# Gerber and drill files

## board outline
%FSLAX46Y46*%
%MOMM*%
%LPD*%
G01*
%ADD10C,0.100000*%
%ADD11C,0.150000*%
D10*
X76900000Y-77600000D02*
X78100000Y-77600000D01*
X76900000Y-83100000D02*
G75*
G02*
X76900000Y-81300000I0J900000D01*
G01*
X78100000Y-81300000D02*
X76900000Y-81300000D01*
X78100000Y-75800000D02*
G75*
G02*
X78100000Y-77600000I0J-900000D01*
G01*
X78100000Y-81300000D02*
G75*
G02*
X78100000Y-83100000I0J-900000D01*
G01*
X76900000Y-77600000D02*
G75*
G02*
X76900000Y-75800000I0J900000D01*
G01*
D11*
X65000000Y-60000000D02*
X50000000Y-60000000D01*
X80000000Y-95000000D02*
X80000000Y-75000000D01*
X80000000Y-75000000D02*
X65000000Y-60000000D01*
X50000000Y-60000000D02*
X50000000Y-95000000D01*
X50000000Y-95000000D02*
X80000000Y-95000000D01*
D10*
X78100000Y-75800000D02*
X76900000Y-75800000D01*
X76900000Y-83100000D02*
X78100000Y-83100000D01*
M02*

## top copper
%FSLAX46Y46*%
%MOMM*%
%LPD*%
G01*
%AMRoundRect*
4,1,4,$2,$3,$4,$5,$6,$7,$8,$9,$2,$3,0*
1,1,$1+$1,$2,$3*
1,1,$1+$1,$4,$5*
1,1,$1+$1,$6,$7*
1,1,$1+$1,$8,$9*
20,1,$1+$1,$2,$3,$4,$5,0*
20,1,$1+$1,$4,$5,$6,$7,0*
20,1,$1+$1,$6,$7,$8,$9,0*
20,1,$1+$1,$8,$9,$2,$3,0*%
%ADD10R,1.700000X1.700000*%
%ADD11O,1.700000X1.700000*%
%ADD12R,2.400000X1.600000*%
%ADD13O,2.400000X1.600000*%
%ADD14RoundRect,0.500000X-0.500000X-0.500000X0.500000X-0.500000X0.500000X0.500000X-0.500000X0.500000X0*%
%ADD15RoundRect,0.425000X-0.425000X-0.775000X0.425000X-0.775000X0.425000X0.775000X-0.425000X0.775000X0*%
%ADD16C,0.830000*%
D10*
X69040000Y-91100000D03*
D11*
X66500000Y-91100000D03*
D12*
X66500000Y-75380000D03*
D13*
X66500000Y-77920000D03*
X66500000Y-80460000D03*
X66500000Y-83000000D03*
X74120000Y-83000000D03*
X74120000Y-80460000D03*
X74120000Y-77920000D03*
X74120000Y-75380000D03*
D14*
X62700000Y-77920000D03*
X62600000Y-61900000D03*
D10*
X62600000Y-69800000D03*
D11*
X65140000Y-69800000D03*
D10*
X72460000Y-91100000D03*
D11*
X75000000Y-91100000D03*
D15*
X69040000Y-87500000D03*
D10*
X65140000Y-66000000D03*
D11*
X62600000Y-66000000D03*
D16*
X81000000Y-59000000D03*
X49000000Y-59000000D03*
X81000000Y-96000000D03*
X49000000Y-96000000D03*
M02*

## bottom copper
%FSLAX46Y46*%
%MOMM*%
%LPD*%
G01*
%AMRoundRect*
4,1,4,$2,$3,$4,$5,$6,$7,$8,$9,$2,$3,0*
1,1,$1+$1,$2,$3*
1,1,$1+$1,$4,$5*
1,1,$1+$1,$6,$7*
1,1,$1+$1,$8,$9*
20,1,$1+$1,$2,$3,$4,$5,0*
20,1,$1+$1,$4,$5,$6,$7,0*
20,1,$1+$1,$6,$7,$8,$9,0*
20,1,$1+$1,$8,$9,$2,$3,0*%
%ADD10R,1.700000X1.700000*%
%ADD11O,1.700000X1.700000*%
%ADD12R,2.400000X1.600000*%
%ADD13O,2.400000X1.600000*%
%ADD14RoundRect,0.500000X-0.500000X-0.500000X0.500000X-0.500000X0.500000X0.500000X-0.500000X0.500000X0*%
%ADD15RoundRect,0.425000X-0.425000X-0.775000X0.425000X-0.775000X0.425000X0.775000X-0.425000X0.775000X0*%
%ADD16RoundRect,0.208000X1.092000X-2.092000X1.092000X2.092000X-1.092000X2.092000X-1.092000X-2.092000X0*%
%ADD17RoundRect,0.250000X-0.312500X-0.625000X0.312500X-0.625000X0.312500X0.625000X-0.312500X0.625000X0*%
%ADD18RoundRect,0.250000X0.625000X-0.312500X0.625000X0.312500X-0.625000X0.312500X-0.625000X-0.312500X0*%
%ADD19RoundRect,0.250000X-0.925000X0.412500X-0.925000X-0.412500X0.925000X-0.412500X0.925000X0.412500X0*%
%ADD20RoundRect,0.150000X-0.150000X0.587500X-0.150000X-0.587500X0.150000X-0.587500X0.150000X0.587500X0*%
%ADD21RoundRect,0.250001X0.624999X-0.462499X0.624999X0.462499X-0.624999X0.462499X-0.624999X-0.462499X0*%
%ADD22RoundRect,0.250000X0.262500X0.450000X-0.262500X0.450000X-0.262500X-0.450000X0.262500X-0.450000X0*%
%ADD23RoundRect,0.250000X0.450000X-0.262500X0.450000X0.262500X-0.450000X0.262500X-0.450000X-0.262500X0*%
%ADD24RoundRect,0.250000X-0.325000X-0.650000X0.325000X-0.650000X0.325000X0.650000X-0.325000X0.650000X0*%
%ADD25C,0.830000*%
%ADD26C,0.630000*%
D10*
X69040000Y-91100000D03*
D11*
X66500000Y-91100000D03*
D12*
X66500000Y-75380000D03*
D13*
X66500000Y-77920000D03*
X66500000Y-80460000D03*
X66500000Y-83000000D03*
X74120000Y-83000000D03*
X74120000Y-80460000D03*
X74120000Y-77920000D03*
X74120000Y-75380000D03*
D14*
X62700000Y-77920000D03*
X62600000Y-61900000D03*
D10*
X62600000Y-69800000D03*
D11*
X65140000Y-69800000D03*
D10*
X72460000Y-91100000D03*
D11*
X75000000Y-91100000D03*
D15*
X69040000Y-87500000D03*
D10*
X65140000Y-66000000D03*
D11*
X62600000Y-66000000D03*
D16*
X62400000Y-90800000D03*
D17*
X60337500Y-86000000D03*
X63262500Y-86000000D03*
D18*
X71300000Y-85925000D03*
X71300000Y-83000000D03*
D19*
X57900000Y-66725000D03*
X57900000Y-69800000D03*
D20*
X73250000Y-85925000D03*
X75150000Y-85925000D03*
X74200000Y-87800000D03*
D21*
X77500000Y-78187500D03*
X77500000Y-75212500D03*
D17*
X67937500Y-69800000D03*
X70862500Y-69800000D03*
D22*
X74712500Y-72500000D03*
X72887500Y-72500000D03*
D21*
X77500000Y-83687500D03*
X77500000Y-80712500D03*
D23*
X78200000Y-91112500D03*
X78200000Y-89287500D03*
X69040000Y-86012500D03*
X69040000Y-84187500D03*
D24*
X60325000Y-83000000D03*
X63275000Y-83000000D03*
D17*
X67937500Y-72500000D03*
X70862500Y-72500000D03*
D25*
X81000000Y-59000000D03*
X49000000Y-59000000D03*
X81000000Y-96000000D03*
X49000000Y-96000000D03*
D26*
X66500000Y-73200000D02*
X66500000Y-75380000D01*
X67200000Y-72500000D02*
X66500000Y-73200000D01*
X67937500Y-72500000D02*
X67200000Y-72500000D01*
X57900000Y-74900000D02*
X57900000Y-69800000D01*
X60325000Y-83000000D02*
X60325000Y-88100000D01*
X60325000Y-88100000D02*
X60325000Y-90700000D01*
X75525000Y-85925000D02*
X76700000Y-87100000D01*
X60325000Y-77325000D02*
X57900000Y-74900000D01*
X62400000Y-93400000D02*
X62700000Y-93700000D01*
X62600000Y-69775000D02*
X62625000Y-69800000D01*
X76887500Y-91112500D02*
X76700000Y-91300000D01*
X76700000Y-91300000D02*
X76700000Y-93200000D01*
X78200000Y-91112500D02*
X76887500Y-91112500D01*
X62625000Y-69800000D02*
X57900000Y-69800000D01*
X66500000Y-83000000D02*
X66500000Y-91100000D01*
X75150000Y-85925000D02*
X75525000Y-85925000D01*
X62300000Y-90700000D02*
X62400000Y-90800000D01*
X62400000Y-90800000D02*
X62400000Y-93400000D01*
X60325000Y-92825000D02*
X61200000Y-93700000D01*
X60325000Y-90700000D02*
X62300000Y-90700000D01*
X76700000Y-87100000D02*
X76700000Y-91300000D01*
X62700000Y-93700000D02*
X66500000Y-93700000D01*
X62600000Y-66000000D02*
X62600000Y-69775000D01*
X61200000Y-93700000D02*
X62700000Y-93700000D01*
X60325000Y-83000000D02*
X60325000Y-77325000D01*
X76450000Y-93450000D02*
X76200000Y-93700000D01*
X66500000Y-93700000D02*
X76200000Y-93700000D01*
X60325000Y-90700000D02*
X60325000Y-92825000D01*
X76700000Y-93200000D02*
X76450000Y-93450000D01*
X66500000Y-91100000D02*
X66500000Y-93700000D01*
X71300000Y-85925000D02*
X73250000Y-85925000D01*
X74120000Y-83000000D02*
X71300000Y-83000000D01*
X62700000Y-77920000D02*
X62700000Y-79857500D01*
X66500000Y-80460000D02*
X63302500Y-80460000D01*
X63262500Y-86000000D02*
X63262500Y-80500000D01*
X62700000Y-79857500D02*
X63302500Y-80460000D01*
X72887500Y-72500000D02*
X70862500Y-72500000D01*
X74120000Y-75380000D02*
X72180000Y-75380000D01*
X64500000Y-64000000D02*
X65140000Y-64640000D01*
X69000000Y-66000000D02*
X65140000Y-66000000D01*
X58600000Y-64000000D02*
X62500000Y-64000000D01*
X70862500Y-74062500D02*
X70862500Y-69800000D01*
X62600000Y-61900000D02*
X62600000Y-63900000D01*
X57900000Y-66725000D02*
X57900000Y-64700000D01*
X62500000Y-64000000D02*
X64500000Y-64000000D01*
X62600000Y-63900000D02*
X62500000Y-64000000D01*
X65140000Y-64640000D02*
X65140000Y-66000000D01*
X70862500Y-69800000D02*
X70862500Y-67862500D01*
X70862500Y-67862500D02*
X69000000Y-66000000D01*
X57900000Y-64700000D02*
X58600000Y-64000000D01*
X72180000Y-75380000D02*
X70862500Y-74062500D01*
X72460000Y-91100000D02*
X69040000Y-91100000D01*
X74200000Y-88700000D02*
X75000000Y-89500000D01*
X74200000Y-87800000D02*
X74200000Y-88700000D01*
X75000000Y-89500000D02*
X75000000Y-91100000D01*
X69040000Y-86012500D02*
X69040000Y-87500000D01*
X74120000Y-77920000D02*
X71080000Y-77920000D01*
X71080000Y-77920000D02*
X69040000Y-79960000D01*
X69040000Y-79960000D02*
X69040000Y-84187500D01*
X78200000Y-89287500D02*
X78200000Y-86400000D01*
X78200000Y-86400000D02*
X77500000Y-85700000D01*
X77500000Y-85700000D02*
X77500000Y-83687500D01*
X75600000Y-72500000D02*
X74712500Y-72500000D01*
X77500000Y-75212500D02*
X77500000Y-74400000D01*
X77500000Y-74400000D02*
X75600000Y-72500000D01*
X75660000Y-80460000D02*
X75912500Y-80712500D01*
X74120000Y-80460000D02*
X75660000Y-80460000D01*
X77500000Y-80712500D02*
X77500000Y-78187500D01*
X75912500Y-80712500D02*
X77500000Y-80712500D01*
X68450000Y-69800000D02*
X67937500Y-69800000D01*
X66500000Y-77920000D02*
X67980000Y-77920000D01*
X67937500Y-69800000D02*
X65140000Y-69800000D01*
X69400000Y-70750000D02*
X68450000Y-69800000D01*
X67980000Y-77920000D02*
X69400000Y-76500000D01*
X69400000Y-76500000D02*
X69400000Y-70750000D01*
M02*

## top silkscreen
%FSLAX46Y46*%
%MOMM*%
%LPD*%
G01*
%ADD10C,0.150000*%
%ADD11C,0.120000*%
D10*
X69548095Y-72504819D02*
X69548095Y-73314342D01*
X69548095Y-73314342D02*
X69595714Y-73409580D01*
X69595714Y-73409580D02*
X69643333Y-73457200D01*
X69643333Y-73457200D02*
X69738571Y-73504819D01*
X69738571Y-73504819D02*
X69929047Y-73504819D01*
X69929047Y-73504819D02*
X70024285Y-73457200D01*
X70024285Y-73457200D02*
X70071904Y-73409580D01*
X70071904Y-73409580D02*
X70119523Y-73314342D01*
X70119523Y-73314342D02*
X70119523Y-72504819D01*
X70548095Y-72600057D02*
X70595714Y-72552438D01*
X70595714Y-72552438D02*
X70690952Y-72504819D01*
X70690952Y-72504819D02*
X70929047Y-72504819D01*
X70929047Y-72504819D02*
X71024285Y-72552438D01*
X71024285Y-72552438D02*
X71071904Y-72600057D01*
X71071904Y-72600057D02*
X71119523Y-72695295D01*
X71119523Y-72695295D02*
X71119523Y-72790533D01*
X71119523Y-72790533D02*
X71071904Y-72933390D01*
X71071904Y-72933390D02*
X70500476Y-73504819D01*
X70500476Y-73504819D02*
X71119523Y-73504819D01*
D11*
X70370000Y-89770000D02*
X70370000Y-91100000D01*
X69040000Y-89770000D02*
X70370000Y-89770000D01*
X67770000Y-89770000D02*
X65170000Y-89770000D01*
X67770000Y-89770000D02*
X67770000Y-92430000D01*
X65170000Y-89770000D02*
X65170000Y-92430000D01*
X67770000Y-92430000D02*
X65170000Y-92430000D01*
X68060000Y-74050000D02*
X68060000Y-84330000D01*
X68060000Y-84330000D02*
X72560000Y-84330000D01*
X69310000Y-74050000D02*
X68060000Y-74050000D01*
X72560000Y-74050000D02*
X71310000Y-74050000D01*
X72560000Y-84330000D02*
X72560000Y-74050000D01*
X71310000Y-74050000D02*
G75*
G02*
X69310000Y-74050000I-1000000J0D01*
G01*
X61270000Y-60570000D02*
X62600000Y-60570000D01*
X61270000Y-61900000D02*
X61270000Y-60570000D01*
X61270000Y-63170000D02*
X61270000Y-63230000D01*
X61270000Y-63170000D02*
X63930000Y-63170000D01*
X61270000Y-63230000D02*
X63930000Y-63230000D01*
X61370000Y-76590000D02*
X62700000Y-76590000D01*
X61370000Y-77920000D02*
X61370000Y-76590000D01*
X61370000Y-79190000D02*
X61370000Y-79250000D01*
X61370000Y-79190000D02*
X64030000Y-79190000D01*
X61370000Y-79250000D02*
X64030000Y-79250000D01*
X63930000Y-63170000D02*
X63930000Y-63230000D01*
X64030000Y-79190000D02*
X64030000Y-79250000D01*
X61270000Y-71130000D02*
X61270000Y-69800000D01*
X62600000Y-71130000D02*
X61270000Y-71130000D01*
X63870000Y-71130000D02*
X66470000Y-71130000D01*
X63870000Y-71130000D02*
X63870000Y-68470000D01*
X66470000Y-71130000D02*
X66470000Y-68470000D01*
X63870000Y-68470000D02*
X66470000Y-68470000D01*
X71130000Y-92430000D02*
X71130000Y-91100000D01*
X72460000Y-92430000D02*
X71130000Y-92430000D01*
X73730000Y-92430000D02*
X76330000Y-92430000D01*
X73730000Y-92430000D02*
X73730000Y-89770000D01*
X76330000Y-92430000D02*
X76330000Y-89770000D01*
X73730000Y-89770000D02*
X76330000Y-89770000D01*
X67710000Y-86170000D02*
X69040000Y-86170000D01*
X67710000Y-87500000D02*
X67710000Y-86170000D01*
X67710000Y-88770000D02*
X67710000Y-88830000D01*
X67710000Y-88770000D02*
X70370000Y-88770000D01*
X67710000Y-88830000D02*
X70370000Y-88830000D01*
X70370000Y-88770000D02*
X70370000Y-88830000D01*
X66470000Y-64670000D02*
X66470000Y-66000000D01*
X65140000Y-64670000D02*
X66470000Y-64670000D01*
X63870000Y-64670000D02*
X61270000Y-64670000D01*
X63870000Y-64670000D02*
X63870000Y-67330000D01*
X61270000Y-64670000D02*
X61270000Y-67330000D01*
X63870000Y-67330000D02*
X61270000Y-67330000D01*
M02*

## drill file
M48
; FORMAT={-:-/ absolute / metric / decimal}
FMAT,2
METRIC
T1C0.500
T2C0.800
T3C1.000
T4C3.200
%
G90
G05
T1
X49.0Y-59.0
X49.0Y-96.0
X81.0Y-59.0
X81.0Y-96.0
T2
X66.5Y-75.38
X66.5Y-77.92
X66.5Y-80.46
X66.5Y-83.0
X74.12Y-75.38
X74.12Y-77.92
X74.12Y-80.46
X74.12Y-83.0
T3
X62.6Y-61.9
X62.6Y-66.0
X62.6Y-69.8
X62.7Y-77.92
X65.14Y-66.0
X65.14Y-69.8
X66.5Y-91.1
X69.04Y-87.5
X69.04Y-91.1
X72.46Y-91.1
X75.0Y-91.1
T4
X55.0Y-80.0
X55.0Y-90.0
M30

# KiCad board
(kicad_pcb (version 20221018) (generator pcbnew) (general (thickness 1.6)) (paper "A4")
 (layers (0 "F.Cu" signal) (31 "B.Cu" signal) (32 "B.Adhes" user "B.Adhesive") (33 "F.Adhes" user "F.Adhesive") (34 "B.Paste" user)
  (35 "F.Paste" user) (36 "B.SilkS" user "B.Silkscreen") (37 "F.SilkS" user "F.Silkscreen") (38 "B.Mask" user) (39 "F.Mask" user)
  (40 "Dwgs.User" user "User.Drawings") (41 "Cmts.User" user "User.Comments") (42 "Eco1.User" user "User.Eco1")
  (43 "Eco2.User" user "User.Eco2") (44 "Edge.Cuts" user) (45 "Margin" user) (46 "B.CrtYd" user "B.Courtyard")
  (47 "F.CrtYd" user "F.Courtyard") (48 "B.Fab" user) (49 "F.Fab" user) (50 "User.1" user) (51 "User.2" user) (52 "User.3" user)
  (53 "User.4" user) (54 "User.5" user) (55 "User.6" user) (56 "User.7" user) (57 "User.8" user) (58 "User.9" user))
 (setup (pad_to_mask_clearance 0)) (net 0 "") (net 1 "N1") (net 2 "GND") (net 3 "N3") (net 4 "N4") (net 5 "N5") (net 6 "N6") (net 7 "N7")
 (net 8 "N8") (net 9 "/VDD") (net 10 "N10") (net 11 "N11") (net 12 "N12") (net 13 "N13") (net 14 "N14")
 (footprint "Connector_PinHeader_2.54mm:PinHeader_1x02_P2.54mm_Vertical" (layer "F.Cu") (at 69.04 91.1 -90)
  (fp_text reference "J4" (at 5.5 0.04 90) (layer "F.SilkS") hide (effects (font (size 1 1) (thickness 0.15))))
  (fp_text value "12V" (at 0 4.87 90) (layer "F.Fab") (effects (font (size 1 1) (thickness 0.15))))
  (fp_line (start -1.33 -1.33) (end 0 -1.33) (stroke (width 0.12) (type solid)) (layer "F.SilkS"))
  (fp_line (start -1.33 0) (end -1.33 -1.33) (stroke (width 0.12) (type solid)) (layer "F.SilkS"))
  (fp_line (start -1.33 1.27) (end -1.33 3.87) (stroke (width 0.12) (type solid)) (layer "F.SilkS"))
  (fp_line (start -1.33 1.27) (end 1.33 1.27) (stroke (width 0.12) (type solid)) (layer "F.SilkS"))
  (fp_line (start -1.33 3.87) (end 1.33 3.87) (stroke (width 0.12) (type solid)) (layer "F.SilkS"))
  (fp_line (start 1.33 1.27) (end 1.33 3.87) (stroke (width 0.12) (type solid)) (layer "F.SilkS"))
  (pad "1" thru_hole rect (at 0 0 270) (size 1.7 1.7) (drill 1) (layers "*.Cu" "*.Mask") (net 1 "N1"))
  (pad "2" thru_hole oval (at 0 2.54 270) (size 1.7 1.7) (drill 1) (layers "*.Cu" "*.Mask") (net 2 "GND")))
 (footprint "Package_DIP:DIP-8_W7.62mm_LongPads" (layer "F.Cu") (at 66.5 75.38)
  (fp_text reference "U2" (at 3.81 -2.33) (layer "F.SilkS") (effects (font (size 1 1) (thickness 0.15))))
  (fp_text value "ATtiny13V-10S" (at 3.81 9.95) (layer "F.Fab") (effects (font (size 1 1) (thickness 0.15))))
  (fp_line (start 1.56 -1.33) (end 1.56 8.95) (stroke (width 0.12) (type solid)) (layer "F.SilkS"))
  (fp_line (start 1.56 8.95) (end 6.06 8.95) (stroke (width 0.12) (type solid)) (layer "F.SilkS"))
  (fp_line (start 2.81 -1.33) (end 1.56 -1.33) (stroke (width 0.12) (type solid)) (layer "F.SilkS"))
  (fp_line (start 6.06 -1.33) (end 4.81 -1.33) (stroke (width 0.12) (type solid)) (layer "F.SilkS"))
  (fp_line (start 6.06 8.95) (end 6.06 -1.33) (stroke (width 0.12) (type solid)) (layer "F.SilkS"))
  (fp_arc (start 4.81 -1.33) (mid 3.81 -0.33) (end 2.81 -1.33) (stroke (width 0.12) (type solid)) (layer "F.SilkS"))
  (pad "1" thru_hole rect (at 0 0) (size 2.4 1.6) (drill 0.8) (layers "*.Cu" "*.Mask") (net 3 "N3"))
  (pad "2" thru_hole oval (at 0 2.54) (size 2.4 1.6) (drill 0.8) (layers "*.Cu" "*.Mask") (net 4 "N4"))
  (pad "3" thru_hole oval (at 0 5.08) (size 2.4 1.6) (drill 0.8) (layers "*.Cu" "*.Mask") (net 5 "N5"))
  (pad "4" thru_hole oval (at 0 7.62) (size 2.4 1.6) (drill 0.8) (layers "*.Cu" "*.Mask") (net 2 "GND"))
  (pad "5" thru_hole oval (at 7.62 7.62) (size 2.4 1.6) (drill 0.8) (layers "*.Cu" "*.Mask") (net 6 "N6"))
  (pad "6" thru_hole oval (at 7.62 5.08) (size 2.4 1.6) (drill 0.8) (layers "*.Cu" "*.Mask") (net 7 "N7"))
  (pad "7" thru_hole oval (at 7.62 2.54) (size 2.4 1.6) (drill 0.8) (layers "*.Cu" "*.Mask") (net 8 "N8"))
  (pad "8" thru_hole oval (at 7.62 0) (size 2.4 1.6) (drill 0.8) (layers "*.Cu" "*.Mask") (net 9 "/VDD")))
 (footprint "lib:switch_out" (layer "F.Cu") (at 62.7 68.92)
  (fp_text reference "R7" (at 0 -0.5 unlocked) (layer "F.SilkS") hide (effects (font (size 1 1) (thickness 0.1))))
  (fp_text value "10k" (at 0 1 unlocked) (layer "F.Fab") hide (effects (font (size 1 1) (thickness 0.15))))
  (fp_line (start -1.43 -8.35) (end -0.1 -8.35) (stroke (width 0.12) (type solid)) (layer "F.SilkS"))
  (fp_line (start -1.43 -7.02) (end -1.43 -8.35) (stroke (width 0.12) (type solid)) (layer "F.SilkS"))
  (fp_line (start -1.43 -5.75) (end -1.43 -5.69) (stroke (width 0.12) (type solid)) (layer "F.SilkS"))
  (fp_line (start -1.43 -5.75) (end 1.23 -5.75) (stroke (width 0.12) (type solid)) (layer "F.SilkS"))
  (fp_line (start -1.43 -5.69) (end 1.23 -5.69) (stroke (width 0.12) (type solid)) (layer "F.SilkS"))
  (fp_line (start -1.33 7.67) (end 0 7.67) (stroke (width 0.12) (type solid)) (layer "F.SilkS"))
  (fp_line (start -1.33 9) (end -1.33 7.67) (stroke (width 0.12) (type solid)) (layer "F.SilkS"))
  (fp_line (start -1.33 10.27) (end -1.33 10.33) (stroke (width 0.12) (type solid)) (layer "F.SilkS"))
  (fp_line (start -1.33 10.27) (end 1.33 10.27) (stroke (width 0.12) (type solid)) (layer "F.SilkS"))
  (fp_line (start -1.33 10.33) (end 1.33 10.33) (stroke (width 0.12) (type solid)) (layer "F.SilkS"))
  (fp_line (start 1.23 -5.75) (end 1.23 -5.69) (stroke (width 0.12) (type solid)) (layer "F.SilkS"))
  (fp_line (start 1.33 10.27) (end 1.33 10.33) (stroke (width 0.12) (type solid)) (layer "F.SilkS"))
  (pad "1" thru_hole roundrect (at 0 9) (size 2 2) (drill 1) (layers "*.Cu" "*.Mask") (roundrect_rratio 0.25) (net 5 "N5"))
  (pad "2" thru_hole roundrect (at -0.1 -7.02) (size 2 2) (drill 1) (layers "*.Cu" "*.Mask") (roundrect_rratio 0.25) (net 9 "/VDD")))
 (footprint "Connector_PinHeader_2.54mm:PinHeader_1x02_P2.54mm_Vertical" (layer "F.Cu") (at 62.6 69.8 90)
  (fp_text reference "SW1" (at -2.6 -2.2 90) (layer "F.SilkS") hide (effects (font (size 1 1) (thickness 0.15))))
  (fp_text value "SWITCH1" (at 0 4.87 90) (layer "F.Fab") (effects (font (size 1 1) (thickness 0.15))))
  (fp_line (start -1.33 -1.33) (end 0 -1.33) (stroke (width 0.12) (type solid)) (layer "F.SilkS"))
  (fp_line (start -1.33 0) (end -1.33 -1.33) (stroke (width 0.12) (type solid)) (layer "F.SilkS"))
  (fp_line (start -1.33 1.27) (end -1.33 3.87) (stroke (width 0.12) (type solid)) (layer "F.SilkS"))
  (fp_line (start -1.33 1.27) (end 1.33 1.27) (stroke (width 0.12) (type solid)) (layer "F.SilkS"))
  (fp_line (start -1.33 3.87) (end 1.33 3.87) (stroke (width 0.12) (type solid)) (layer "F.SilkS"))
  (fp_line (start 1.33 1.27) (end 1.33 3.87) (stroke (width 0.12) (type solid)) (layer "F.SilkS"))
  (pad "1" thru_hole rect (at 0 0 90) (size 1.7 1.7) (drill 1) (layers "*.Cu" "*.Mask") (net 2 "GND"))
  (pad "2" thru_hole oval (at 0 2.54 90) (size 1.7 1.7) (drill 1) (layers "*.Cu" "*.Mask") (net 4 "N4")))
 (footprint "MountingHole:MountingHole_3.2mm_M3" (layer "F.Cu") (at 55 90)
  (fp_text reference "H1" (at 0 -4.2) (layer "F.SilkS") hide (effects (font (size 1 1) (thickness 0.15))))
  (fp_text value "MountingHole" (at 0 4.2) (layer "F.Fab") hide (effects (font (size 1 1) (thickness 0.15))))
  (pad "" np_thru_hole circle (at 0 0) (size 3.2 3.2) (drill 3.2) (layers "*.Cu" "*.Mask")))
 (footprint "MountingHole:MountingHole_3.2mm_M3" (layer "F.Cu") (at 55 80)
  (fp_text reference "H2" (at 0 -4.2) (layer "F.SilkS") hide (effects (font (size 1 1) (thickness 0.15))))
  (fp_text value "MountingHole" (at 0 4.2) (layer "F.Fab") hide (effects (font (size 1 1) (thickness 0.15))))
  (pad "" np_thru_hole circle (at 0 0) (size 3.2 3.2) (drill 3.2) (layers "*.Cu" "*.Mask")))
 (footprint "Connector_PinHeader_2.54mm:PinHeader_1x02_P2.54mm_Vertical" (layer "F.Cu") (at 72.46 91.1 90)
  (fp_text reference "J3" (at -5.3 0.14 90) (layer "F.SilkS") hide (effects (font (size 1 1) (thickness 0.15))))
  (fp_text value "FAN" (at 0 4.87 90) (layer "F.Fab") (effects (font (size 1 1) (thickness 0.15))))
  (fp_line (start -1.33 -1.33) (end 0 -1.33) (stroke (width 0.12) (type solid)) (layer "F.SilkS"))
  (fp_line (start -1.33 0) (end -1.33 -1.33) (stroke (width 0.12) (type solid)) (layer "F.SilkS"))
  (fp_line (start -1.33 1.27) (end -1.33 3.87) (stroke (width 0.12) (type solid)) (layer "F.SilkS"))
  (fp_line (start -1.33 1.27) (end 1.33 1.27) (stroke (width 0.12) (type solid)) (layer "F.SilkS"))
  (fp_line (start -1.33 3.87) (end 1.33 3.87) (stroke (width 0.12) (type solid)) (layer "F.SilkS"))
  (fp_line (start 1.33 1.27) (end 1.33 3.87) (stroke (width 0.12) (type solid)) (layer "F.SilkS"))
  (pad "1" thru_hole rect (at 0 0 90) (size 1.7 1.7) (drill 1) (layers "*.Cu" "*.Mask") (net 1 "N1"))
  (pad "2" thru_hole oval (at 0 2.54 90) (size 1.7 1.7) (drill 1) (layers "*.Cu" "*.Mask") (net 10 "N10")))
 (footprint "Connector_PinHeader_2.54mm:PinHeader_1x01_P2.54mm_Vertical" (layer "F.Cu") (at 69.04 87.5)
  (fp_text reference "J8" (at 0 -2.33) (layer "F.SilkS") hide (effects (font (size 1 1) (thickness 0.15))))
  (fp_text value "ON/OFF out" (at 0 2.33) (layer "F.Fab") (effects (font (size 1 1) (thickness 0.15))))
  (fp_line (start -1.33 -1.33) (end 0 -1.33) (stroke (width 0.12) (type solid)) (layer "F.SilkS"))
  (fp_line (start -1.33 0) (end -1.33 -1.33) (stroke (width 0.12) (type solid)) (layer "F.SilkS"))
  (fp_line (start -1.33 1.27) (end -1.33 1.33) (stroke (width 0.12) (type solid)) (layer "F.SilkS"))
  (fp_line (start -1.33 1.27) (end 1.33 1.27) (stroke (width 0.12) (type solid)) (layer "F.SilkS"))
  (fp_line (start -1.33 1.33) (end 1.33 1.33) (stroke (width 0.12) (type solid)) (layer "F.SilkS"))
  (fp_line (start 1.33 1.27) (end 1.33 1.33) (stroke (width 0.12) (type solid)) (layer "F.SilkS"))
  (pad "1" thru_hole roundrect (at 0 0) (size 1.7 2.4) (drill 1) (layers "*.Cu" "*.Mask") (roundrect_rratio 0.25) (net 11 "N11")))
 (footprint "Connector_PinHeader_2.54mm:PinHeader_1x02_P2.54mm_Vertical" (layer "F.Cu") (at 65.14 66 -90)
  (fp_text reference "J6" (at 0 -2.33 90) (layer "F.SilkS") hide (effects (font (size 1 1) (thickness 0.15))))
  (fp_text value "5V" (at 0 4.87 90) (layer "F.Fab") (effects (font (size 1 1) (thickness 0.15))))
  (fp_line (start -1.33 -1.33) (end 0 -1.33) (stroke (width 0.12) (type solid)) (layer "F.SilkS"))
  (fp_line (start -1.33 0) (end -1.33 -1.33) (stroke (width 0.12) (type solid)) (layer "F.SilkS"))
  (fp_line (start -1.33 1.27) (end -1.33 3.87) (stroke (width 0.12) (type solid)) (layer "F.SilkS"))
  (fp_line (start -1.33 1.27) (end 1.33 1.27) (stroke (width 0.12) (type solid)) (layer "F.SilkS"))
  (fp_line (start -1.33 3.87) (end 1.33 3.87) (stroke (width 0.12) (type solid)) (layer "F.SilkS"))
  (fp_line (start 1.33 1.27) (end 1.33 3.87) (stroke (width 0.12) (type solid)) (layer "F.SilkS"))
  (pad "1" thru_hole rect (at 0 0 270) (size 1.7 1.7) (drill 1) (layers "*.Cu" "*.Mask") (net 9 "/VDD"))
  (pad "2" thru_hole oval (at 0 2.54 270) (size 1.7 1.7) (drill 1) (layers "*.Cu" "*.Mask") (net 2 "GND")))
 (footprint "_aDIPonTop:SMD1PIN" (layer "B.Cu") (at 62.4 90.8 90)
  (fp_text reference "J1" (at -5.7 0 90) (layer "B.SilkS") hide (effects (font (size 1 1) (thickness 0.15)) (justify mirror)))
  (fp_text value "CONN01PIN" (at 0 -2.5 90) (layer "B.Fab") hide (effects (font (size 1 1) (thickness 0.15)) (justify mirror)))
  (pad "1" smd roundrect (at 0 0 90) (size 4.6 2.6) (layers "B.Cu" "B.Paste" "B.Mask") (roundrect_rratio 0.08) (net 2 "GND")))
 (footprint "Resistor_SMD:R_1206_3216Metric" (layer "B.Cu") (at 61.8 86)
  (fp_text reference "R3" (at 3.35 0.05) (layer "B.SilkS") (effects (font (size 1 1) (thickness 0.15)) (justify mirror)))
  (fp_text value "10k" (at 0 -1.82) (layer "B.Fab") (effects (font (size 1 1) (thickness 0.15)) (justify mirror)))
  (pad "1" smd roundrect (at -1.4625 0) (size 1.125 1.75) (layers "B.Cu" "B.Paste" "B.Mask") (roundrect_rratio 0.2222222222) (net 2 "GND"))
  (pad "2" smd roundrect (at 1.4625 0) (size 1.125 1.75) (layers "B.Cu" "B.Paste" "B.Mask") (roundrect_rratio 0.2222222222) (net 5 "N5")))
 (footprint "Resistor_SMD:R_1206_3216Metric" (layer "B.Cu") (at 71.3 84.4625 90)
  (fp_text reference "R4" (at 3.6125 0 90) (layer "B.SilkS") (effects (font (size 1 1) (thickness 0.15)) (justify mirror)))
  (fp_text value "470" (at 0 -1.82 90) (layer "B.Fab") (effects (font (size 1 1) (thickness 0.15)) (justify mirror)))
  (pad "1" smd roundrect (at -1.4625 0 90) (size 1.125 1.75) (layers "B.Cu" "B.Paste" "B.Mask") (roundrect_rratio 0.2222222222)
   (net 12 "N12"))
  (pad "2" smd roundrect (at 1.4625 0 90) (size 1.125 1.75) (layers "B.Cu" "B.Paste" "B.Mask") (roundrect_rratio 0.2222222222) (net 6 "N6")))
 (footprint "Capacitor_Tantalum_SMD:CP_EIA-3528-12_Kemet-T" (layer "B.Cu") (at 57.9 68.2625 -90)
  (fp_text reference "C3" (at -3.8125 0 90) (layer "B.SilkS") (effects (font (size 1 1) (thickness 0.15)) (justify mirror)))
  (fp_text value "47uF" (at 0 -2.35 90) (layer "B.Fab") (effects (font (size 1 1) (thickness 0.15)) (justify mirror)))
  (pad "1" smd roundrect (at -1.5375 0 270) (size 1.325 2.35) (layers "B.Cu" "B.Paste" "B.Mask") (roundrect_rratio 0.1886792453)
   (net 9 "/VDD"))
  (pad "2" smd roundrect (at 1.5375 0 270) (size 1.325 2.35) (layers "B.Cu" "B.Paste" "B.Mask") (roundrect_rratio 0.1886792453)
   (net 2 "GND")))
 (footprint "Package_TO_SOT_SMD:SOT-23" (layer "B.Cu") (at 74.2 86.8625 -90)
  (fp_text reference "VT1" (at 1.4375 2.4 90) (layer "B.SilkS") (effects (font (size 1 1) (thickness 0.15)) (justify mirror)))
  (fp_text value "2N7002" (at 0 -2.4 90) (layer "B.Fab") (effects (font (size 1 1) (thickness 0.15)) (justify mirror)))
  (pad "1" smd roundrect (at -0.9375 0.95 270) (size 1.475 0.6) (layers "B.Cu" "B.Paste" "B.Mask") (roundrect_rratio 0.25) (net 12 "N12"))
  (pad "2" smd roundrect (at -0.9375 -0.95 270) (size 1.475 0.6) (layers "B.Cu" "B.Paste" "B.Mask") (roundrect_rratio 0.25) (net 2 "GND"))
  (pad "3" smd roundrect (at 0.9375 0 270) (size 1.475 0.6) (layers "B.Cu" "B.Paste" "B.Mask") (roundrect_rratio 0.25) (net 10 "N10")))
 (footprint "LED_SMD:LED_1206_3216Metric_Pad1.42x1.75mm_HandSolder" (layer "B.Cu") (at 77.5 76.7 90)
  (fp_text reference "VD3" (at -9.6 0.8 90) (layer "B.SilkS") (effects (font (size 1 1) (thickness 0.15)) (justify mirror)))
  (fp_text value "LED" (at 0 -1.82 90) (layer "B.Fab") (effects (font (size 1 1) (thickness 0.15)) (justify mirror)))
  (pad "1" smd roundrect (at -1.4875 0 90) (size 1.425 1.75) (layers "B.Cu" "B.Paste" "B.Mask") (roundrect_rratio 0.1754392982) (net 7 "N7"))
  (pad "2" smd roundrect (at 1.4875 0 90) (size 1.425 1.75) (layers "B.Cu" "B.Paste" "B.Mask") (roundrect_rratio 0.1754392982)
   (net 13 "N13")))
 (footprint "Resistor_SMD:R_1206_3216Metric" (layer "B.Cu") (at 69.4 69.8)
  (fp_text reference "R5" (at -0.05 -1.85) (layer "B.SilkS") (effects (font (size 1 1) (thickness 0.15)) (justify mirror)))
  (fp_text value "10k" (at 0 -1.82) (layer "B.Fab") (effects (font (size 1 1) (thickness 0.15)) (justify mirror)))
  (pad "1" smd roundrect (at -1.4625 0) (size 1.125 1.75) (layers "B.Cu" "B.Paste" "B.Mask") (roundrect_rratio 0.2222222222) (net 4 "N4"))
  (pad "2" smd roundrect (at 1.4625 0) (size 1.125 1.75) (layers "B.Cu" "B.Paste" "B.Mask") (roundrect_rratio 0.2222222222) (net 9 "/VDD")))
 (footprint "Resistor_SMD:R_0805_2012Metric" (layer "B.Cu") (at 73.8 72.5 180)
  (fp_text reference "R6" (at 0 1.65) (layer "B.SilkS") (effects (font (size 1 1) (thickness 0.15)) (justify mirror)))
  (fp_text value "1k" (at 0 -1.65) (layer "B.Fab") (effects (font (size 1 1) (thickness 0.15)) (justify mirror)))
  (pad "1" smd roundrect (at -0.9125 0 180) (size 1.025 1.4) (layers "B.Cu" "B.Paste" "B.Mask") (roundrect_rratio 0.243902439)
   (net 13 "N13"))
  (pad "2" smd roundrect (at 0.9125 0 180) (size 1.025 1.4) (layers "B.Cu" "B.Paste" "B.Mask") (roundrect_rratio 0.243902439) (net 9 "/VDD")))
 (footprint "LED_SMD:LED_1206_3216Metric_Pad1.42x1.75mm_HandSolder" (layer "B.Cu") (at 77.5 82.2 90)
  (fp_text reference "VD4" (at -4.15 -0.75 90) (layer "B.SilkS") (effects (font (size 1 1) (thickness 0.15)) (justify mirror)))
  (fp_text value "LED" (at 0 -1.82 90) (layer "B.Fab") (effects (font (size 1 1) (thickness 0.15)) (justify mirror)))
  (pad "1" smd roundrect (at -1.4875 0 90) (size 1.425 1.75) (layers "B.Cu" "B.Paste" "B.Mask") (roundrect_rratio 0.1754392982)
   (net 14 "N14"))
  (pad "2" smd roundrect (at 1.4875 0 90) (size 1.425 1.75) (layers "B.Cu" "B.Paste" "B.Mask") (roundrect_rratio 0.1754392982) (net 7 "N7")))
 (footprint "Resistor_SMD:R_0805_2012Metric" (layer "B.Cu") (at 78.2 90.2 90)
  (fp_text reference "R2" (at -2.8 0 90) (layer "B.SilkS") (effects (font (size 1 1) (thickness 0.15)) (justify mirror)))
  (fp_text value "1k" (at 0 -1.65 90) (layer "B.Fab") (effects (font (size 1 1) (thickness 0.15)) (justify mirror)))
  (pad "1" smd roundrect (at -0.9125 0 90) (size 1.025 1.4) (layers "B.Cu" "B.Paste" "B.Mask") (roundrect_rratio 0.243902439) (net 2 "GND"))
  (pad "2" smd roundrect (at 0.9125 0 90) (size 1.025 1.4) (layers "B.Cu" "B.Paste" "B.Mask") (roundrect_rratio 0.243902439) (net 14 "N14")))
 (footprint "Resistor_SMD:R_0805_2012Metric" (layer "B.Cu") (at 69.04 85.1 90)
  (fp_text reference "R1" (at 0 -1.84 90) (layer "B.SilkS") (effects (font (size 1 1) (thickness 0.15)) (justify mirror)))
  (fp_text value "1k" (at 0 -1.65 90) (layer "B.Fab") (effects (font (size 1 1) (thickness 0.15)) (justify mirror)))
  (pad "1" smd roundrect (at -0.9125 0 90) (size 1.025 1.4) (layers "B.Cu" "B.Paste" "B.Mask") (roundrect_rratio 0.243902439) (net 11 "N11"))
  (pad "2" smd roundrect (at 0.9125 0 90) (size 1.025 1.4) (layers "B.Cu" "B.Paste" "B.Mask") (roundrect_rratio 0.243902439) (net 8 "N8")))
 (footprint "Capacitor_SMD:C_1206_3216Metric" (layer "B.Cu") (at 61.8 83)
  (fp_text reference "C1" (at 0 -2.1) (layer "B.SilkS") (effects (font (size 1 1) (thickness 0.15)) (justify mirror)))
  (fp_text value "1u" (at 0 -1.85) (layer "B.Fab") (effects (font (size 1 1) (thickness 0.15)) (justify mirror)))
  (pad "1" smd roundrect (at -1.475 0) (size 1.15 1.8) (layers "B.Cu" "B.Paste" "B.Mask") (roundrect_rratio 0.2173913043) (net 2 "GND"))
  (pad "2" smd roundrect (at 1.475 0) (size 1.15 1.8) (layers "B.Cu" "B.Paste" "B.Mask") (roundrect_rratio 0.2173913043) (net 5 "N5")))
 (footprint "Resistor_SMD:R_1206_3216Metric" (layer "B.Cu") (at 69.4 72.5)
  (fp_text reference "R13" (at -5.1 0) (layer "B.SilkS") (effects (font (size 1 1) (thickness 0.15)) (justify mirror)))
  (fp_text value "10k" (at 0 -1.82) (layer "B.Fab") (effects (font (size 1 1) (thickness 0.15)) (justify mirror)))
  (pad "1" smd roundrect (at -1.4625 0) (size 1.125 1.75) (layers "B.Cu" "B.Paste" "B.Mask") (roundrect_rratio 0.2222222222) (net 3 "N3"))
  (pad "2" smd roundrect (at 1.4625 0) (size 1.125 1.75) (layers "B.Cu" "B.Paste" "B.Mask") (roundrect_rratio 0.2222222222) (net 9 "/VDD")))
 (gr_line (start 76.9 77.6) (end 78.1 77.6) (stroke (width 0.1) (type default)) (layer "Edge.Cuts"))
 (gr_arc (start 76.9 83.1) (mid 76 82.2) (end 76.9 81.3) (stroke (width 0.1) (type default)) (layer "Edge.Cuts"))
 (gr_line (start 78.1 81.3) (end 76.9 81.3) (stroke (width 0.1) (type default)) (layer "Edge.Cuts"))
 (gr_arc (start 78.1 75.8) (mid 79 76.7) (end 78.1 77.6) (stroke (width 0.1) (type default)) (layer "Edge.Cuts"))
 (gr_arc (start 78.1 81.3) (mid 79 82.2) (end 78.1 83.1) (stroke (width 0.1) (type default)) (layer "Edge.Cuts"))
 (gr_arc (start 76.9 77.6) (mid 76 76.7) (end 76.9 75.8) (stroke (width 0.1) (type default)) (layer "Edge.Cuts"))
 (gr_line (start 65 60) (end 50 60) (stroke (width 0.15) (type default)) (layer "Edge.Cuts"))
 (gr_line (start 80 95) (end 80 75) (stroke (width 0.15) (type default)) (layer "Edge.Cuts"))
 (gr_line (start 80 75) (end 65 60) (stroke (width 0.15) (type default)) (layer "Edge.Cuts"))
 (gr_line (start 50 60) (end 50 95) (stroke (width 0.15) (type default)) (layer "Edge.Cuts"))
 (gr_line (start 50 95) (end 80 95) (stroke (width 0.15) (type default)) (layer "Edge.Cuts"))
 (gr_line (start 78.1 75.8) (end 76.9 75.8) (stroke (width 0.1) (type default)) (layer "Edge.Cuts"))
 (gr_line (start 76.9 83.1) (end 78.1 83.1) (stroke (width 0.1) (type default)) (layer "Edge.Cuts"))
 (via (at 81 59) (size 0.83) (drill 0.5) (layers "F.Cu" "B.Cu") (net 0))
 (via (at 49 59) (size 0.83) (drill 0.5) (layers "F.Cu" "B.Cu") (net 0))
 (via (at 81 96) (size 0.83) (drill 0.5) (layers "F.Cu" "B.Cu") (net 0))
 (via (at 49 96) (size 0.83) (drill 0.5) (layers "F.Cu" "B.Cu") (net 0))
 (segment (start 66.5 73.2) (end 66.5 75.38) (width 0.63) (layer "B.Cu") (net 3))
 (segment (start 67.2 72.5) (end 66.5 73.2) (width 0.63) (layer "B.Cu") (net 3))
 (segment (start 67.9375 72.5) (end 67.2 72.5) (width 0.63) (layer "B.Cu") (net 3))
 (segment (start 57.9 74.9) (end 57.9 69.8) (width 0.63) (layer "B.Cu") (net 2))
 (segment (start 60.325 83) (end 60.325 88.1) (width 0.63) (layer "B.Cu") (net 2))
 (segment (start 60.325 88.1) (end 60.325 90.7) (width 0.63) (layer "B.Cu") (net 2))
 (segment (start 75.525 85.925) (end 76.7 87.1) (width 0.63) (layer "B.Cu") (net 2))
 (segment (start 60.325 77.325) (end 57.9 74.9) (width 0.63) (layer "B.Cu") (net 2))
 (segment (start 62.4 93.4) (end 62.7 93.7) (width 0.63) (layer "B.Cu") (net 2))
 (segment (start 62.6 69.775) (end 62.625 69.8) (width 0.63) (layer "B.Cu") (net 2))
 (segment (start 76.8875 91.1125) (end 76.7 91.3) (width 0.63) (layer "B.Cu") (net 2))
 (segment (start 76.7 91.3) (end 76.7 93.2) (width 0.63) (layer "B.Cu") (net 2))
 (segment (start 78.2 91.1125) (end 76.8875 91.1125) (width 0.63) (layer "B.Cu") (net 2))
 (segment (start 62.625 69.8) (end 57.9 69.8) (width 0.63) (layer "B.Cu") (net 2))
 (segment (start 66.5 83) (end 66.5 91.1) (width 0.63) (layer "B.Cu") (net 2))
 (segment (start 75.15 85.925) (end 75.525 85.925) (width 0.63) (layer "B.Cu") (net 2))
 (segment (start 62.3 90.7) (end 62.4 90.8) (width 0.63) (layer "B.Cu") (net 2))
 (segment (start 62.4 90.8) (end 62.4 93.4) (width 0.63) (layer "B.Cu") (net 2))
 (segment (start 60.325 92.825) (end 61.2 93.7) (width 0.63) (layer "B.Cu") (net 2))
 (segment (start 60.325 90.7) (end 62.3 90.7) (width 0.63) (layer "B.Cu") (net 2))
 (segment (start 76.7 87.1) (end 76.7 91.3) (width 0.63) (layer "B.Cu") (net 2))
 (segment (start 62.7 93.7) (end 66.5 93.7) (width 0.63) (layer "B.Cu") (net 2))
 (segment (start 62.6 66) (end 62.6 69.775) (width 0.63) (layer "B.Cu") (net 2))
 (segment (start 61.2 93.7) (end 62.7 93.7) (width 0.63) (layer "B.Cu") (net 2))
 (segment (start 60.325 83) (end 60.325 77.325) (width 0.63) (layer "B.Cu") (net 2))
 (segment (start 76.45 93.45) (end 76.2 93.7) (width 0.63) (layer "B.Cu") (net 2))
 (segment (start 66.5 93.7) (end 76.2 93.7) (width 0.63) (layer "B.Cu") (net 2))
 (segment (start 60.325 90.7) (end 60.325 92.825) (width 0.63) (layer "B.Cu") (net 2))
 (segment (start 76.7 93.2) (end 76.45 93.45) (width 0.63) (layer "B.Cu") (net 2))
 (segment (start 66.5 91.1) (end 66.5 93.7) (width 0.63) (layer "B.Cu") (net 2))
 (segment (start 71.3 85.925) (end 73.25 85.925) (width 0.63) (layer "B.Cu") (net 12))
 (segment (start 74.12 83) (end 71.3 83) (width 0.63) (layer "B.Cu") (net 6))
 (segment (start 62.7 77.92) (end 62.7 79.8575) (width 0.63) (layer "B.Cu") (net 5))
 (segment (start 66.5 80.46) (end 63.3025 80.46) (width 0.63) (layer "B.Cu") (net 5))
 (segment (start 63.2625 86) (end 63.2625 80.5) (width 0.63) (layer "B.Cu") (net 5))
 (segment (start 62.7 79.8575) (end 63.3025 80.46) (width 0.63) (layer "B.Cu") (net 5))
 (segment (start 72.8875 72.5) (end 70.8625 72.5) (width 0.63) (layer "B.Cu") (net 9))
 (segment (start 74.12 75.38) (end 72.18 75.38) (width 0.63) (layer "B.Cu") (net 9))
 (segment (start 64.5 64) (end 65.14 64.64) (width 0.63) (layer "B.Cu") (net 9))
 (segment (start 69 66) (end 65.14 66) (width 0.63) (layer "B.Cu") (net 9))
 (segment (start 58.6 64) (end 62.5 64) (width 0.63) (layer "B.Cu") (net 9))
 (segment (start 70.8625 74.0625) (end 70.8625 69.8) (width 0.63) (layer "B.Cu") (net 9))
 (segment (start 62.6 61.9) (end 62.6 63.9) (width 0.63) (layer "B.Cu") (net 9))
 (segment (start 57.9 66.725) (end 57.9 64.7) (width 0.63) (layer "B.Cu") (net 9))
 (segment (start 62.5 64) (end 64.5 64) (width 0.63) (layer "B.Cu") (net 9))
 (segment (start 62.6 63.9) (end 62.5 64) (width 0.63) (layer "B.Cu") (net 9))
 (segment (start 65.14 64.64) (end 65.14 66) (width 0.63) (layer "B.Cu") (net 9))
 (segment (start 70.8625 69.8) (end 70.8625 67.8625) (width 0.63) (layer "B.Cu") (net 9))
 (segment (start 70.8625 67.8625) (end 69 66) (width 0.63) (layer "B.Cu") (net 9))
 (segment (start 57.9 64.7) (end 58.6 64) (width 0.63) (layer "B.Cu") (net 9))
 (segment (start 72.18 75.38) (end 70.8625 74.0625) (width 0.63) (layer "B.Cu") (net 9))
 (segment (start 72.46 91.1) (end 69.04 91.1) (width 0.63) (layer "B.Cu") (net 1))
 (segment (start 74.2 88.7) (end 75 89.5) (width 0.63) (layer "B.Cu") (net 10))
 (segment (start 74.2 87.8) (end 74.2 88.7) (width 0.63) (layer "B.Cu") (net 10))
 (segment (start 75 89.5) (end 75 91.1) (width 0.63) (layer "B.Cu") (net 10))
 (segment (start 69.04 86.0125) (end 69.04 87.5) (width 0.63) (layer "B.Cu") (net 11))
 (segment (start 74.12 77.92) (end 71.08 77.92) (width 0.63) (layer "B.Cu") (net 8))
 (segment (start 71.08 77.92) (end 69.04 79.96) (width 0.63) (layer "B.Cu") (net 8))
 (segment (start 69.04 79.96) (end 69.04 84.1875) (width 0.63) (layer "B.Cu") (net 8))
 (segment (start 78.2 89.2875) (end 78.2 86.4) (width 0.63) (layer "B.Cu") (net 14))
 (segment (start 78.2 86.4) (end 77.5 85.7) (width 0.63) (layer "B.Cu") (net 14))
 (segment (start 77.5 85.7) (end 77.5 83.6875) (width 0.63) (layer "B.Cu") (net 14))
 (segment (start 75.6 72.5) (end 74.7125 72.5) (width 0.63) (layer "B.Cu") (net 13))
 (segment (start 77.5 75.2125) (end 77.5 74.4) (width 0.63) (layer "B.Cu") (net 13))
 (segment (start 77.5 74.4) (end 75.6 72.5) (width 0.63) (layer "B.Cu") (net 13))
 (segment (start 75.66 80.46) (end 75.9125 80.7125) (width 0.63) (layer "B.Cu") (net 7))
 (segment (start 74.12 80.46) (end 75.66 80.46) (width 0.63) (layer "B.Cu") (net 7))
 (segment (start 77.5 80.7125) (end 77.5 78.1875) (width 0.63) (layer "B.Cu") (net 7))
 (segment (start 75.9125 80.7125) (end 77.5 80.7125) (width 0.63) (layer "B.Cu") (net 7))
 (segment (start 68.45 69.8) (end 67.9375 69.8) (width 0.63) (layer "B.Cu") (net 4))
 (segment (start 66.5 77.92) (end 67.98 77.92) (width 0.63) (layer "B.Cu") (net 4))
 (segment (start 67.9375 69.8) (end 65.14 69.8) (width 0.63) (layer "B.Cu") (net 4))
 (segment (start 69.4 70.75) (end 68.45 69.8) (width 0.63) (layer "B.Cu") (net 4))
 (segment (start 67.98 77.92) (end 69.4 76.5) (width 0.63) (layer "B.Cu") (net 4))
 (segment (start 69.4 76.5) (end 69.4 70.75) (width 0.63) (layer "B.Cu") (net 4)))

